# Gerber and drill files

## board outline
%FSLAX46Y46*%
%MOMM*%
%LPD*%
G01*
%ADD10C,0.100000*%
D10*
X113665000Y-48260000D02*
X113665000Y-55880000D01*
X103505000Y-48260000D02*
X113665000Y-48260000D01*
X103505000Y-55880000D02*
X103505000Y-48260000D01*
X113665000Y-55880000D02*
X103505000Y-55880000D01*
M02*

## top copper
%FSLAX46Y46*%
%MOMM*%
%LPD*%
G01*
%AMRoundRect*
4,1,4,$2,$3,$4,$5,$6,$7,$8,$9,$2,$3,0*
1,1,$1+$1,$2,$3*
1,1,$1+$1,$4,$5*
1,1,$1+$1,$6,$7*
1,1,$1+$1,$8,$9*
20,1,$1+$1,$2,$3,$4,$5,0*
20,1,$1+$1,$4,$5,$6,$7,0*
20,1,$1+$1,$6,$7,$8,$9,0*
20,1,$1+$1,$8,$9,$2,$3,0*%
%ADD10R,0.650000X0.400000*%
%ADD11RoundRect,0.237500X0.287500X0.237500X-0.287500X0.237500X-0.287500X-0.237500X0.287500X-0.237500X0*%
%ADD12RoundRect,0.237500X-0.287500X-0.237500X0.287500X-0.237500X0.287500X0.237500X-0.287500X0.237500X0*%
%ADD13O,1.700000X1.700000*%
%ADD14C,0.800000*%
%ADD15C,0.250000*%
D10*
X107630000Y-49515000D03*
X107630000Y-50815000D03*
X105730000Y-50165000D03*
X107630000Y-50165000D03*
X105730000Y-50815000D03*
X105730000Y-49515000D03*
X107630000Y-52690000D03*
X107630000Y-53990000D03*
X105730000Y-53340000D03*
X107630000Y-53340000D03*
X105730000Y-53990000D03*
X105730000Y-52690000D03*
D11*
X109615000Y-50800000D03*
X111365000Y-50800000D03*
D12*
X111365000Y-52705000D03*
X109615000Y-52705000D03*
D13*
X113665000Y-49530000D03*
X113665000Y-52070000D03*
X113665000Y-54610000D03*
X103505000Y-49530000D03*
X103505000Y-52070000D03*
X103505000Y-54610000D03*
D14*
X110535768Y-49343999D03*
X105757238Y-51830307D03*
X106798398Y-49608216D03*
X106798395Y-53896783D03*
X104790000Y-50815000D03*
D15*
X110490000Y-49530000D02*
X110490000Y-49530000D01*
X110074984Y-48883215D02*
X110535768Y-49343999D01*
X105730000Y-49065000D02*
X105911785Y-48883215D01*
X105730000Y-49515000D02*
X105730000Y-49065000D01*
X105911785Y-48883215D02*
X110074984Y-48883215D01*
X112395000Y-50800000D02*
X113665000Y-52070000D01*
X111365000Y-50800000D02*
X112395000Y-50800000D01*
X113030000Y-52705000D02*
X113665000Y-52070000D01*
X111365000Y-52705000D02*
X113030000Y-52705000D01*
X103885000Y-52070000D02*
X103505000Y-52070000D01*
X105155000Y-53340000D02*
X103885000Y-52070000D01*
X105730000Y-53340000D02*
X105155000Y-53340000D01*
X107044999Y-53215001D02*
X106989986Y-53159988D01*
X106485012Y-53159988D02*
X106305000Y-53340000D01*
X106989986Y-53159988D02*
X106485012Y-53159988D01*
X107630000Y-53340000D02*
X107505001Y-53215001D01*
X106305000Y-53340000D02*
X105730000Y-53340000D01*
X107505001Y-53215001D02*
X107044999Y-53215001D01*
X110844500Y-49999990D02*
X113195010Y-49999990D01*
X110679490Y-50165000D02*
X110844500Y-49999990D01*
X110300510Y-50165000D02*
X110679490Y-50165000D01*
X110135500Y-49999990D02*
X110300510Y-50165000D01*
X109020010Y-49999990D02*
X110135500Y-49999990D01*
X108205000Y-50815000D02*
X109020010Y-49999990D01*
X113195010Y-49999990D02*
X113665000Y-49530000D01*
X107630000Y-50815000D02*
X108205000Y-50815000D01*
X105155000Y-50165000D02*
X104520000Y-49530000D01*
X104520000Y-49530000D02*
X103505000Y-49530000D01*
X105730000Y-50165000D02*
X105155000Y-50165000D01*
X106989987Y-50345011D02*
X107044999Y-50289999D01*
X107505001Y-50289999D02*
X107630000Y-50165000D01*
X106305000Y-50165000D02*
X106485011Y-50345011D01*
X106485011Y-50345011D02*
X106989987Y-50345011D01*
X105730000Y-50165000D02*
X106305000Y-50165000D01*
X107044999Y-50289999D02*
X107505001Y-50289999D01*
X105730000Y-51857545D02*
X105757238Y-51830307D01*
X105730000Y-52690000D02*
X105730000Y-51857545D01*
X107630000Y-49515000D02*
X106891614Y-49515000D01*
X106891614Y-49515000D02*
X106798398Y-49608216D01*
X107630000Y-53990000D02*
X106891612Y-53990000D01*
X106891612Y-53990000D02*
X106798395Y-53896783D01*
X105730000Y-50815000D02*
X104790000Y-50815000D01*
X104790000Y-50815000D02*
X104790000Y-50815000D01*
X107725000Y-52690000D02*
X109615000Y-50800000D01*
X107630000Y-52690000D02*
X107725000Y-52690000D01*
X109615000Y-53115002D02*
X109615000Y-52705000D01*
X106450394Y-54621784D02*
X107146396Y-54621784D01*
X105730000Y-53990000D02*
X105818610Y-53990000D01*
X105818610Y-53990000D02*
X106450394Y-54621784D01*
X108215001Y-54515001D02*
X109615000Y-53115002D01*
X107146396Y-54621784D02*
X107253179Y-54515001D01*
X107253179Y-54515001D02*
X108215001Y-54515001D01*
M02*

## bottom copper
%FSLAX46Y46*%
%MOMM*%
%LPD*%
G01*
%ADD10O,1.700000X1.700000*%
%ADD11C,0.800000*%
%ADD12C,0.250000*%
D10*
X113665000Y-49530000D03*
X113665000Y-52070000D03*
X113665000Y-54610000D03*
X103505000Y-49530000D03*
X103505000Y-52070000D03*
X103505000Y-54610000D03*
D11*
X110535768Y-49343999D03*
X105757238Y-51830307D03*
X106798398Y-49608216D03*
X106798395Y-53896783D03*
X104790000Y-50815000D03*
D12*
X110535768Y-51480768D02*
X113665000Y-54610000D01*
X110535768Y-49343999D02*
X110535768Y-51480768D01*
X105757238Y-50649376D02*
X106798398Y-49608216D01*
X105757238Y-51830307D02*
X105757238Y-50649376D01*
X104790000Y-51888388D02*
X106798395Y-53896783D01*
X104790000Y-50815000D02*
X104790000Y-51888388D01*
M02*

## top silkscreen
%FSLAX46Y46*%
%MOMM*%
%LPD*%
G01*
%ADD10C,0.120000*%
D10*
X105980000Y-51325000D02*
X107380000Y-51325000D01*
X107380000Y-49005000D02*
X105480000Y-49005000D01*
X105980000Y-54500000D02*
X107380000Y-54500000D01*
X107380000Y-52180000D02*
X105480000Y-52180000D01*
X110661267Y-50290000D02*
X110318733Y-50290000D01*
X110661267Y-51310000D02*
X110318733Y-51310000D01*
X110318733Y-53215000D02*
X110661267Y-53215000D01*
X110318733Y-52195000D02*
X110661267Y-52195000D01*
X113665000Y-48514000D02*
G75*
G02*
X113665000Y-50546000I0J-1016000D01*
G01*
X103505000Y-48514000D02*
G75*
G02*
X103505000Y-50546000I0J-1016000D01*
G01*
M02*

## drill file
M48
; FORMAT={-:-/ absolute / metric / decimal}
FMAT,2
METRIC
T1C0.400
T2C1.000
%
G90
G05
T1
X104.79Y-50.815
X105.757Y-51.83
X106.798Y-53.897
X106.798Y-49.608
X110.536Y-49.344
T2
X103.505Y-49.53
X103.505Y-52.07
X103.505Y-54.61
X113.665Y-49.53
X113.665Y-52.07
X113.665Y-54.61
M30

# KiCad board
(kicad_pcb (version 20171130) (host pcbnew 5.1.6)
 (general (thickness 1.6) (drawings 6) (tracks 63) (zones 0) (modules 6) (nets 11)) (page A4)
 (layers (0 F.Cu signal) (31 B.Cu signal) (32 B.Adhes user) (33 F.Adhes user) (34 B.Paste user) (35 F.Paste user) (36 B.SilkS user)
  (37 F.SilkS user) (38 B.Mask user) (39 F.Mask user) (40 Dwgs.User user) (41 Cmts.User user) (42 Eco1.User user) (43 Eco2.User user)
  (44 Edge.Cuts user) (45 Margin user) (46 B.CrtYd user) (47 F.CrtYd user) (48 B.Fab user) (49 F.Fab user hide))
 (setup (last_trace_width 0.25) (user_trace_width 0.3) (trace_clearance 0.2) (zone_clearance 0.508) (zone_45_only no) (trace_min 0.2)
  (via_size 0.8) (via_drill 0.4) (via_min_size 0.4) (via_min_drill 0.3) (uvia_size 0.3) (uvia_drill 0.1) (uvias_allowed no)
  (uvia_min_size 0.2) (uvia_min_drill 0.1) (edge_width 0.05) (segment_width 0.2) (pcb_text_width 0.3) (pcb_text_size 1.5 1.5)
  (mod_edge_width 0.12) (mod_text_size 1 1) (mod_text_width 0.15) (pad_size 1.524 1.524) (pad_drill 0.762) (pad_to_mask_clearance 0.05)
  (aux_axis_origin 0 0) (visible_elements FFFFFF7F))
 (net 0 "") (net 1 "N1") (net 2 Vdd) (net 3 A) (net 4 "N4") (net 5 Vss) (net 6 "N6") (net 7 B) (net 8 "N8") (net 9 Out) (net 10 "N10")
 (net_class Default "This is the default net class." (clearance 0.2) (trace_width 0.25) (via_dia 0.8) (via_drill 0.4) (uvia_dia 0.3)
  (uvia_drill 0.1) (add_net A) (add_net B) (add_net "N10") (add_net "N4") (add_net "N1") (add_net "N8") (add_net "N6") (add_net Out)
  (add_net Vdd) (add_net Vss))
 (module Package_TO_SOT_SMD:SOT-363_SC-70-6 (layer F.Cu) (at 106.68 50.165)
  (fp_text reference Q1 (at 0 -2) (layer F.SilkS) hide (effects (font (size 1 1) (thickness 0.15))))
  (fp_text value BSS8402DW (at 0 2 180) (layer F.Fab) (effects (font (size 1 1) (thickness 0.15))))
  (fp_line (start -0.7 1.16) (end 0.7 1.16) (layer F.SilkS) (width 0.12))
  (fp_line (start 0.7 -1.16) (end -1.2 -1.16) (layer F.SilkS) (width 0.12))
  (pad 6 smd rect (at 0.95 -0.65) (size 0.65 0.4) (layers F.Cu F.Paste F.Mask) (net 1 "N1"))
  (pad 4 smd rect (at 0.95 0.65) (size 0.65 0.4) (layers F.Cu F.Paste F.Mask) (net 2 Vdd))
  (pad 2 smd rect (at -0.95 0) (size 0.65 0.4) (layers F.Cu F.Paste F.Mask) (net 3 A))
  (pad 5 smd rect (at 0.95 0) (size 0.65 0.4) (layers F.Cu F.Paste F.Mask) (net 3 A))
  (pad 3 smd rect (at -0.95 0.65) (size 0.65 0.4) (layers F.Cu F.Paste F.Mask) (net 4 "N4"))
  (pad 1 smd rect (at -0.95 -0.65) (size 0.65 0.4) (layers F.Cu F.Paste F.Mask) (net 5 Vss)))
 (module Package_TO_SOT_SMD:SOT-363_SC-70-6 (layer F.Cu) (at 106.68 53.34)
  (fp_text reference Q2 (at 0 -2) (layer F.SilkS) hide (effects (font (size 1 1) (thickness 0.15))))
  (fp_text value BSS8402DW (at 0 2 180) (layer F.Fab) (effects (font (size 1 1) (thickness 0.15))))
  (fp_line (start -0.7 1.16) (end 0.7 1.16) (layer F.SilkS) (width 0.12))
  (fp_line (start 0.7 -1.16) (end -1.2 -1.16) (layer F.SilkS) (width 0.12))
  (pad 6 smd rect (at 0.95 -0.65) (size 0.65 0.4) (layers F.Cu F.Paste F.Mask) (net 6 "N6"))
  (pad 4 smd rect (at 0.95 0.65) (size 0.65 0.4) (layers F.Cu F.Paste F.Mask) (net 4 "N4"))
  (pad 2 smd rect (at -0.95 0) (size 0.65 0.4) (layers F.Cu F.Paste F.Mask) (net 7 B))
  (pad 5 smd rect (at 0.95 0) (size 0.65 0.4) (layers F.Cu F.Paste F.Mask) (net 7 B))
  (pad 3 smd rect (at -0.95 0.65) (size 0.65 0.4) (layers F.Cu F.Paste F.Mask) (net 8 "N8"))
  (pad 1 smd rect (at -0.95 -0.65) (size 0.65 0.4) (layers F.Cu F.Paste F.Mask) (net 1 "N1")))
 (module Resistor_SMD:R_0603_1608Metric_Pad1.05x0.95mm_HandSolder (layer F.Cu) (at 110.49 50.8 180)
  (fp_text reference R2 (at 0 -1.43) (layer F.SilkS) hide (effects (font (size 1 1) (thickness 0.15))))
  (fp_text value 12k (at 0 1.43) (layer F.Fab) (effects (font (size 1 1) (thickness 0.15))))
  (fp_line (start -0.171267 0.51) (end 0.171267 0.51) (layer F.SilkS) (width 0.12))
  (fp_line (start -0.171267 -0.51) (end 0.171267 -0.51) (layer F.SilkS) (width 0.12))
  (pad 2 smd roundrect (at 0.875 0 180) (size 1.05 0.95) (layers F.Cu F.Paste F.Mask) (roundrect_rratio 0.25) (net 6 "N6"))
  (pad 1 smd roundrect (at -0.875 0 180) (size 1.05 0.95) (layers F.Cu F.Paste F.Mask) (roundrect_rratio 0.25) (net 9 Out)))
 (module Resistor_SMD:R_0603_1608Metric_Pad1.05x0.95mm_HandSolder (layer F.Cu) (at 110.49 52.705)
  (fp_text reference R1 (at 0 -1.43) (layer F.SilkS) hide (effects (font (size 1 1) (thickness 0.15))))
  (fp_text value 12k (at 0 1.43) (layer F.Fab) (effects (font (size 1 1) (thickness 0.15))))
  (fp_line (start -0.171267 0.51) (end 0.171267 0.51) (layer F.SilkS) (width 0.12))
  (fp_line (start -0.171267 -0.51) (end 0.171267 -0.51) (layer F.SilkS) (width 0.12))
  (pad 2 smd roundrect (at 0.875 0) (size 1.05 0.95) (layers F.Cu F.Paste F.Mask) (roundrect_rratio 0.25) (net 9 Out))
  (pad 1 smd roundrect (at -0.875 0) (size 1.05 0.95) (layers F.Cu F.Paste F.Mask) (roundrect_rratio 0.25) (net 8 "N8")))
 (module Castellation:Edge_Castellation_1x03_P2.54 (layer F.Cu) (at 113.665 49.53)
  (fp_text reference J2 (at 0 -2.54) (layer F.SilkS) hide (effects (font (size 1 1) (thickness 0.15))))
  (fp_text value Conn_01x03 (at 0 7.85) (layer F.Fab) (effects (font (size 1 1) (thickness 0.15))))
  (fp_arc (start 0 0) (end 0 1.016) (angle -180) (layer F.SilkS) (width 0.12))
  (pad 1 thru_hole oval (at 0 0) (size 1.7 1.7) (drill 1) (layers *.Cu *.Mask) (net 2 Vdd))
  (pad 2 thru_hole oval (at 0 2.54) (size 1.7 1.7) (drill 1) (layers *.Cu *.Mask) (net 9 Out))
  (pad 3 thru_hole oval (at 0 5.08) (size 1.7 1.7) (drill 1) (layers *.Cu *.Mask) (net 5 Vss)))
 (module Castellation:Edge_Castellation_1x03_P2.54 (layer F.Cu) (at 103.505 49.53)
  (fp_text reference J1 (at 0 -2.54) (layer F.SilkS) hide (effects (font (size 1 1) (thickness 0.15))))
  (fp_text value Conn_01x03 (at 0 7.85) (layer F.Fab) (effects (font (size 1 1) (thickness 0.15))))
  (fp_arc (start 0 0) (end 0 1.016) (angle -180) (layer F.SilkS) (width 0.12))
  (pad 1 thru_hole oval (at 0 0) (size 1.7 1.7) (drill 1) (layers *.Cu *.Mask) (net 3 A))
  (pad 2 thru_hole oval (at 0 2.54) (size 1.7 1.7) (drill 1) (layers *.Cu *.Mask) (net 7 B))
  (pad 3 thru_hole oval (at 0 5.08) (size 1.7 1.7) (drill 1) (layers *.Cu *.Mask) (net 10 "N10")))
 (gr_line (start 113.665 48.26) (end 113.665 55.88) (layer Edge.Cuts) (width 0.1))
 (gr_line (start 103.505 48.26) (end 113.665 48.26) (layer Edge.Cuts) (width 0.1))
 (gr_line (start 103.505 55.88) (end 103.505 48.26) (layer Edge.Cuts) (width 0.1))
 (gr_line (start 113.665 55.88) (end 103.505 55.88) (layer Edge.Cuts) (width 0.1))
 (segment (start 110.49 49.53) (end 110.49 49.53) (width 0.25) (layer F.Cu) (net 5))
 (via (at 110.535768 49.343999) (size 0.8) (drill 0.4) (layers F.Cu B.Cu) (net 5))
 (segment (start 110.074984 48.883215) (end 110.535768 49.343999) (width 0.25) (layer F.Cu) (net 5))
 (segment (start 105.73 49.065) (end 105.911785 48.883215) (width 0.25) (layer F.Cu) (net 5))
 (segment (start 105.73 49.515) (end 105.73 49.065) (width 0.25) (layer F.Cu) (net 5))
 (segment (start 105.911785 48.883215) (end 110.074984 48.883215) (width 0.25) (layer F.Cu) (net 5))
 (segment (start 110.535768 51.480768) (end 113.665 54.61) (width 0.25) (layer B.Cu) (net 5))
 (segment (start 110.535768 49.343999) (end 110.535768 51.480768) (width 0.25) (layer B.Cu) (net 5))
 (segment (start 112.395 50.8) (end 113.665 52.07) (width 0.25) (layer F.Cu) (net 9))
 (segment (start 111.365 50.8) (end 112.395 50.8) (width 0.25) (layer F.Cu) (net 9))
 (segment (start 113.03 52.705) (end 113.665 52.07) (width 0.25) (layer F.Cu) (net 9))
 (segment (start 111.365 52.705) (end 113.03 52.705) (width 0.25) (layer F.Cu) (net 9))
 (segment (start 103.885 52.07) (end 103.505 52.07) (width 0.25) (layer F.Cu) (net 7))
 (segment (start 105.155 53.34) (end 103.885 52.07) (width 0.25) (layer F.Cu) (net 7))
 (segment (start 105.73 53.34) (end 105.155 53.34) (width 0.25) (layer F.Cu) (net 7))
 (segment (start 107.044999 53.215001) (end 106.989986 53.159988) (width 0.25) (layer F.Cu) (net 7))
 (segment (start 106.485012 53.159988) (end 106.305 53.34) (width 0.25) (layer F.Cu) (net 7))
 (segment (start 106.989986 53.159988) (end 106.485012 53.159988) (width 0.25) (layer F.Cu) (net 7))
 (segment (start 107.63 53.34) (end 107.505001 53.215001) (width 0.25) (layer F.Cu) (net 7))
 (segment (start 106.305 53.34) (end 105.73 53.34) (width 0.25) (layer F.Cu) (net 7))
 (segment (start 107.505001 53.215001) (end 107.044999 53.215001) (width 0.25) (layer F.Cu) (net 7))
 (segment (start 110.8445 49.99999) (end 113.19501 49.99999) (width 0.25) (layer F.Cu) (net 2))
 (segment (start 110.67949 50.165) (end 110.8445 49.99999) (width 0.25) (layer F.Cu) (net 2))
 (segment (start 110.30051 50.165) (end 110.67949 50.165) (width 0.25) (layer F.Cu) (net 2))
 (segment (start 110.1355 49.99999) (end 110.30051 50.165) (width 0.25) (layer F.Cu) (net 2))
 (segment (start 109.02001 49.99999) (end 110.1355 49.99999) (width 0.25) (layer F.Cu) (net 2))
 (segment (start 108.205 50.815) (end 109.02001 49.99999) (width 0.25) (layer F.Cu) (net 2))
 (segment (start 113.19501 49.99999) (end 113.665 49.53) (width 0.25) (layer F.Cu) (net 2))
 (segment (start 107.63 50.815) (end 108.205 50.815) (width 0.25) (layer F.Cu) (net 2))
 (segment (start 105.155 50.165) (end 104.52 49.53) (width 0.25) (layer F.Cu) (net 3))
 (segment (start 104.52 49.53) (end 103.505 49.53) (width 0.25) (layer F.Cu) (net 3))
 (segment (start 105.73 50.165) (end 105.155 50.165) (width 0.25) (layer F.Cu) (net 3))
 (segment (start 106.989987 50.345011) (end 107.044999 50.289999) (width 0.25) (layer F.Cu) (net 3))
 (segment (start 107.505001 50.289999) (end 107.63 50.165) (width 0.25) (layer F.Cu) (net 3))
 (segment (start 106.305 50.165) (end 106.485011 50.345011) (width 0.25) (layer F.Cu) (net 3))
 (segment (start 106.485011 50.345011) (end 106.989987 50.345011) (width 0.25) (layer F.Cu) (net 3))
 (segment (start 105.73 50.165) (end 106.305 50.165) (width 0.25) (layer F.Cu) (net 3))
 (segment (start 107.044999 50.289999) (end 107.505001 50.289999) (width 0.25) (layer F.Cu) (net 3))
 (via (at 105.757238 51.830307) (size 0.8) (drill 0.4) (layers F.Cu B.Cu) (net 1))
 (segment (start 105.73 51.857545) (end 105.757238 51.830307) (width 0.25) (layer F.Cu) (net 1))
 (segment (start 105.73 52.69) (end 105.73 51.857545) (width 0.25) (layer F.Cu) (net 1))
 (segment (start 107.63 49.515) (end 106.891614 49.515) (width 0.25) (layer F.Cu) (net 1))
 (segment (start 105.757238 50.649376) (end 106.798398 49.608216) (width 0.25) (layer B.Cu) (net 1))
 (segment (start 105.757238 51.830307) (end 105.757238 50.649376) (width 0.25) (layer B.Cu) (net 1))
 (via (at 106.798398 49.608216) (size 0.8) (drill 0.4) (layers F.Cu B.Cu) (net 1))
 (segment (start 106.891614 49.515) (end 106.798398 49.608216) (width 0.25) (layer F.Cu) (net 1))
 (segment (start 107.63 53.99) (end 106.891612 53.99) (width 0.25) (layer F.Cu) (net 4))
 (via (at 106.798395 53.896783) (size 0.8) (drill 0.4) (layers F.Cu B.Cu) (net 4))
 (segment (start 106.891612 53.99) (end 106.798395 53.896783) (width 0.25) (layer F.Cu) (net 4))
 (segment (start 105.73 50.815) (end 104.79 50.815) (width 0.25) (layer F.Cu) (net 4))
 (segment (start 104.79 50.815) (end 104.79 50.815) (width 0.25) (layer F.Cu) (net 4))
 (via (at 104.79 50.815) (size 0.8) (drill 0.4) (layers F.Cu B.Cu) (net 4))
 (segment (start 104.79 51.888388) (end 106.798395 53.896783) (width 0.25) (layer B.Cu) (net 4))
 (segment (start 104.79 50.815) (end 104.79 51.888388) (width 0.25) (layer B.Cu) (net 4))
 (segment (start 107.725 52.69) (end 109.615 50.8) (width 0.25) (layer F.Cu) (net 6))
 (segment (start 107.63 52.69) (end 107.725 52.69) (width 0.25) (layer F.Cu) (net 6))
 (segment (start 109.615 53.115002) (end 109.615 52.705) (width 0.25) (layer F.Cu) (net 8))
 (segment (start 106.450394 54.621784) (end 107.146396 54.621784) (width 0.25) (layer F.Cu) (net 8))
 (segment (start 105.73 53.99) (end 105.81861 53.99) (width 0.25) (layer F.Cu) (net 8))
 (segment (start 105.81861 53.99) (end 106.450394 54.621784) (width 0.25) (layer F.Cu) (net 8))
 (segment (start 108.215001 54.515001) (end 109.615 53.115002) (width 0.25) (layer F.Cu) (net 8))
 (segment (start 107.146396 54.621784) (end 107.253179 54.515001) (width 0.25) (layer F.Cu) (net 8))
 (segment (start 107.253179 54.515001) (end 108.215001 54.515001) (width 0.25) (layer F.Cu) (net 8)))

